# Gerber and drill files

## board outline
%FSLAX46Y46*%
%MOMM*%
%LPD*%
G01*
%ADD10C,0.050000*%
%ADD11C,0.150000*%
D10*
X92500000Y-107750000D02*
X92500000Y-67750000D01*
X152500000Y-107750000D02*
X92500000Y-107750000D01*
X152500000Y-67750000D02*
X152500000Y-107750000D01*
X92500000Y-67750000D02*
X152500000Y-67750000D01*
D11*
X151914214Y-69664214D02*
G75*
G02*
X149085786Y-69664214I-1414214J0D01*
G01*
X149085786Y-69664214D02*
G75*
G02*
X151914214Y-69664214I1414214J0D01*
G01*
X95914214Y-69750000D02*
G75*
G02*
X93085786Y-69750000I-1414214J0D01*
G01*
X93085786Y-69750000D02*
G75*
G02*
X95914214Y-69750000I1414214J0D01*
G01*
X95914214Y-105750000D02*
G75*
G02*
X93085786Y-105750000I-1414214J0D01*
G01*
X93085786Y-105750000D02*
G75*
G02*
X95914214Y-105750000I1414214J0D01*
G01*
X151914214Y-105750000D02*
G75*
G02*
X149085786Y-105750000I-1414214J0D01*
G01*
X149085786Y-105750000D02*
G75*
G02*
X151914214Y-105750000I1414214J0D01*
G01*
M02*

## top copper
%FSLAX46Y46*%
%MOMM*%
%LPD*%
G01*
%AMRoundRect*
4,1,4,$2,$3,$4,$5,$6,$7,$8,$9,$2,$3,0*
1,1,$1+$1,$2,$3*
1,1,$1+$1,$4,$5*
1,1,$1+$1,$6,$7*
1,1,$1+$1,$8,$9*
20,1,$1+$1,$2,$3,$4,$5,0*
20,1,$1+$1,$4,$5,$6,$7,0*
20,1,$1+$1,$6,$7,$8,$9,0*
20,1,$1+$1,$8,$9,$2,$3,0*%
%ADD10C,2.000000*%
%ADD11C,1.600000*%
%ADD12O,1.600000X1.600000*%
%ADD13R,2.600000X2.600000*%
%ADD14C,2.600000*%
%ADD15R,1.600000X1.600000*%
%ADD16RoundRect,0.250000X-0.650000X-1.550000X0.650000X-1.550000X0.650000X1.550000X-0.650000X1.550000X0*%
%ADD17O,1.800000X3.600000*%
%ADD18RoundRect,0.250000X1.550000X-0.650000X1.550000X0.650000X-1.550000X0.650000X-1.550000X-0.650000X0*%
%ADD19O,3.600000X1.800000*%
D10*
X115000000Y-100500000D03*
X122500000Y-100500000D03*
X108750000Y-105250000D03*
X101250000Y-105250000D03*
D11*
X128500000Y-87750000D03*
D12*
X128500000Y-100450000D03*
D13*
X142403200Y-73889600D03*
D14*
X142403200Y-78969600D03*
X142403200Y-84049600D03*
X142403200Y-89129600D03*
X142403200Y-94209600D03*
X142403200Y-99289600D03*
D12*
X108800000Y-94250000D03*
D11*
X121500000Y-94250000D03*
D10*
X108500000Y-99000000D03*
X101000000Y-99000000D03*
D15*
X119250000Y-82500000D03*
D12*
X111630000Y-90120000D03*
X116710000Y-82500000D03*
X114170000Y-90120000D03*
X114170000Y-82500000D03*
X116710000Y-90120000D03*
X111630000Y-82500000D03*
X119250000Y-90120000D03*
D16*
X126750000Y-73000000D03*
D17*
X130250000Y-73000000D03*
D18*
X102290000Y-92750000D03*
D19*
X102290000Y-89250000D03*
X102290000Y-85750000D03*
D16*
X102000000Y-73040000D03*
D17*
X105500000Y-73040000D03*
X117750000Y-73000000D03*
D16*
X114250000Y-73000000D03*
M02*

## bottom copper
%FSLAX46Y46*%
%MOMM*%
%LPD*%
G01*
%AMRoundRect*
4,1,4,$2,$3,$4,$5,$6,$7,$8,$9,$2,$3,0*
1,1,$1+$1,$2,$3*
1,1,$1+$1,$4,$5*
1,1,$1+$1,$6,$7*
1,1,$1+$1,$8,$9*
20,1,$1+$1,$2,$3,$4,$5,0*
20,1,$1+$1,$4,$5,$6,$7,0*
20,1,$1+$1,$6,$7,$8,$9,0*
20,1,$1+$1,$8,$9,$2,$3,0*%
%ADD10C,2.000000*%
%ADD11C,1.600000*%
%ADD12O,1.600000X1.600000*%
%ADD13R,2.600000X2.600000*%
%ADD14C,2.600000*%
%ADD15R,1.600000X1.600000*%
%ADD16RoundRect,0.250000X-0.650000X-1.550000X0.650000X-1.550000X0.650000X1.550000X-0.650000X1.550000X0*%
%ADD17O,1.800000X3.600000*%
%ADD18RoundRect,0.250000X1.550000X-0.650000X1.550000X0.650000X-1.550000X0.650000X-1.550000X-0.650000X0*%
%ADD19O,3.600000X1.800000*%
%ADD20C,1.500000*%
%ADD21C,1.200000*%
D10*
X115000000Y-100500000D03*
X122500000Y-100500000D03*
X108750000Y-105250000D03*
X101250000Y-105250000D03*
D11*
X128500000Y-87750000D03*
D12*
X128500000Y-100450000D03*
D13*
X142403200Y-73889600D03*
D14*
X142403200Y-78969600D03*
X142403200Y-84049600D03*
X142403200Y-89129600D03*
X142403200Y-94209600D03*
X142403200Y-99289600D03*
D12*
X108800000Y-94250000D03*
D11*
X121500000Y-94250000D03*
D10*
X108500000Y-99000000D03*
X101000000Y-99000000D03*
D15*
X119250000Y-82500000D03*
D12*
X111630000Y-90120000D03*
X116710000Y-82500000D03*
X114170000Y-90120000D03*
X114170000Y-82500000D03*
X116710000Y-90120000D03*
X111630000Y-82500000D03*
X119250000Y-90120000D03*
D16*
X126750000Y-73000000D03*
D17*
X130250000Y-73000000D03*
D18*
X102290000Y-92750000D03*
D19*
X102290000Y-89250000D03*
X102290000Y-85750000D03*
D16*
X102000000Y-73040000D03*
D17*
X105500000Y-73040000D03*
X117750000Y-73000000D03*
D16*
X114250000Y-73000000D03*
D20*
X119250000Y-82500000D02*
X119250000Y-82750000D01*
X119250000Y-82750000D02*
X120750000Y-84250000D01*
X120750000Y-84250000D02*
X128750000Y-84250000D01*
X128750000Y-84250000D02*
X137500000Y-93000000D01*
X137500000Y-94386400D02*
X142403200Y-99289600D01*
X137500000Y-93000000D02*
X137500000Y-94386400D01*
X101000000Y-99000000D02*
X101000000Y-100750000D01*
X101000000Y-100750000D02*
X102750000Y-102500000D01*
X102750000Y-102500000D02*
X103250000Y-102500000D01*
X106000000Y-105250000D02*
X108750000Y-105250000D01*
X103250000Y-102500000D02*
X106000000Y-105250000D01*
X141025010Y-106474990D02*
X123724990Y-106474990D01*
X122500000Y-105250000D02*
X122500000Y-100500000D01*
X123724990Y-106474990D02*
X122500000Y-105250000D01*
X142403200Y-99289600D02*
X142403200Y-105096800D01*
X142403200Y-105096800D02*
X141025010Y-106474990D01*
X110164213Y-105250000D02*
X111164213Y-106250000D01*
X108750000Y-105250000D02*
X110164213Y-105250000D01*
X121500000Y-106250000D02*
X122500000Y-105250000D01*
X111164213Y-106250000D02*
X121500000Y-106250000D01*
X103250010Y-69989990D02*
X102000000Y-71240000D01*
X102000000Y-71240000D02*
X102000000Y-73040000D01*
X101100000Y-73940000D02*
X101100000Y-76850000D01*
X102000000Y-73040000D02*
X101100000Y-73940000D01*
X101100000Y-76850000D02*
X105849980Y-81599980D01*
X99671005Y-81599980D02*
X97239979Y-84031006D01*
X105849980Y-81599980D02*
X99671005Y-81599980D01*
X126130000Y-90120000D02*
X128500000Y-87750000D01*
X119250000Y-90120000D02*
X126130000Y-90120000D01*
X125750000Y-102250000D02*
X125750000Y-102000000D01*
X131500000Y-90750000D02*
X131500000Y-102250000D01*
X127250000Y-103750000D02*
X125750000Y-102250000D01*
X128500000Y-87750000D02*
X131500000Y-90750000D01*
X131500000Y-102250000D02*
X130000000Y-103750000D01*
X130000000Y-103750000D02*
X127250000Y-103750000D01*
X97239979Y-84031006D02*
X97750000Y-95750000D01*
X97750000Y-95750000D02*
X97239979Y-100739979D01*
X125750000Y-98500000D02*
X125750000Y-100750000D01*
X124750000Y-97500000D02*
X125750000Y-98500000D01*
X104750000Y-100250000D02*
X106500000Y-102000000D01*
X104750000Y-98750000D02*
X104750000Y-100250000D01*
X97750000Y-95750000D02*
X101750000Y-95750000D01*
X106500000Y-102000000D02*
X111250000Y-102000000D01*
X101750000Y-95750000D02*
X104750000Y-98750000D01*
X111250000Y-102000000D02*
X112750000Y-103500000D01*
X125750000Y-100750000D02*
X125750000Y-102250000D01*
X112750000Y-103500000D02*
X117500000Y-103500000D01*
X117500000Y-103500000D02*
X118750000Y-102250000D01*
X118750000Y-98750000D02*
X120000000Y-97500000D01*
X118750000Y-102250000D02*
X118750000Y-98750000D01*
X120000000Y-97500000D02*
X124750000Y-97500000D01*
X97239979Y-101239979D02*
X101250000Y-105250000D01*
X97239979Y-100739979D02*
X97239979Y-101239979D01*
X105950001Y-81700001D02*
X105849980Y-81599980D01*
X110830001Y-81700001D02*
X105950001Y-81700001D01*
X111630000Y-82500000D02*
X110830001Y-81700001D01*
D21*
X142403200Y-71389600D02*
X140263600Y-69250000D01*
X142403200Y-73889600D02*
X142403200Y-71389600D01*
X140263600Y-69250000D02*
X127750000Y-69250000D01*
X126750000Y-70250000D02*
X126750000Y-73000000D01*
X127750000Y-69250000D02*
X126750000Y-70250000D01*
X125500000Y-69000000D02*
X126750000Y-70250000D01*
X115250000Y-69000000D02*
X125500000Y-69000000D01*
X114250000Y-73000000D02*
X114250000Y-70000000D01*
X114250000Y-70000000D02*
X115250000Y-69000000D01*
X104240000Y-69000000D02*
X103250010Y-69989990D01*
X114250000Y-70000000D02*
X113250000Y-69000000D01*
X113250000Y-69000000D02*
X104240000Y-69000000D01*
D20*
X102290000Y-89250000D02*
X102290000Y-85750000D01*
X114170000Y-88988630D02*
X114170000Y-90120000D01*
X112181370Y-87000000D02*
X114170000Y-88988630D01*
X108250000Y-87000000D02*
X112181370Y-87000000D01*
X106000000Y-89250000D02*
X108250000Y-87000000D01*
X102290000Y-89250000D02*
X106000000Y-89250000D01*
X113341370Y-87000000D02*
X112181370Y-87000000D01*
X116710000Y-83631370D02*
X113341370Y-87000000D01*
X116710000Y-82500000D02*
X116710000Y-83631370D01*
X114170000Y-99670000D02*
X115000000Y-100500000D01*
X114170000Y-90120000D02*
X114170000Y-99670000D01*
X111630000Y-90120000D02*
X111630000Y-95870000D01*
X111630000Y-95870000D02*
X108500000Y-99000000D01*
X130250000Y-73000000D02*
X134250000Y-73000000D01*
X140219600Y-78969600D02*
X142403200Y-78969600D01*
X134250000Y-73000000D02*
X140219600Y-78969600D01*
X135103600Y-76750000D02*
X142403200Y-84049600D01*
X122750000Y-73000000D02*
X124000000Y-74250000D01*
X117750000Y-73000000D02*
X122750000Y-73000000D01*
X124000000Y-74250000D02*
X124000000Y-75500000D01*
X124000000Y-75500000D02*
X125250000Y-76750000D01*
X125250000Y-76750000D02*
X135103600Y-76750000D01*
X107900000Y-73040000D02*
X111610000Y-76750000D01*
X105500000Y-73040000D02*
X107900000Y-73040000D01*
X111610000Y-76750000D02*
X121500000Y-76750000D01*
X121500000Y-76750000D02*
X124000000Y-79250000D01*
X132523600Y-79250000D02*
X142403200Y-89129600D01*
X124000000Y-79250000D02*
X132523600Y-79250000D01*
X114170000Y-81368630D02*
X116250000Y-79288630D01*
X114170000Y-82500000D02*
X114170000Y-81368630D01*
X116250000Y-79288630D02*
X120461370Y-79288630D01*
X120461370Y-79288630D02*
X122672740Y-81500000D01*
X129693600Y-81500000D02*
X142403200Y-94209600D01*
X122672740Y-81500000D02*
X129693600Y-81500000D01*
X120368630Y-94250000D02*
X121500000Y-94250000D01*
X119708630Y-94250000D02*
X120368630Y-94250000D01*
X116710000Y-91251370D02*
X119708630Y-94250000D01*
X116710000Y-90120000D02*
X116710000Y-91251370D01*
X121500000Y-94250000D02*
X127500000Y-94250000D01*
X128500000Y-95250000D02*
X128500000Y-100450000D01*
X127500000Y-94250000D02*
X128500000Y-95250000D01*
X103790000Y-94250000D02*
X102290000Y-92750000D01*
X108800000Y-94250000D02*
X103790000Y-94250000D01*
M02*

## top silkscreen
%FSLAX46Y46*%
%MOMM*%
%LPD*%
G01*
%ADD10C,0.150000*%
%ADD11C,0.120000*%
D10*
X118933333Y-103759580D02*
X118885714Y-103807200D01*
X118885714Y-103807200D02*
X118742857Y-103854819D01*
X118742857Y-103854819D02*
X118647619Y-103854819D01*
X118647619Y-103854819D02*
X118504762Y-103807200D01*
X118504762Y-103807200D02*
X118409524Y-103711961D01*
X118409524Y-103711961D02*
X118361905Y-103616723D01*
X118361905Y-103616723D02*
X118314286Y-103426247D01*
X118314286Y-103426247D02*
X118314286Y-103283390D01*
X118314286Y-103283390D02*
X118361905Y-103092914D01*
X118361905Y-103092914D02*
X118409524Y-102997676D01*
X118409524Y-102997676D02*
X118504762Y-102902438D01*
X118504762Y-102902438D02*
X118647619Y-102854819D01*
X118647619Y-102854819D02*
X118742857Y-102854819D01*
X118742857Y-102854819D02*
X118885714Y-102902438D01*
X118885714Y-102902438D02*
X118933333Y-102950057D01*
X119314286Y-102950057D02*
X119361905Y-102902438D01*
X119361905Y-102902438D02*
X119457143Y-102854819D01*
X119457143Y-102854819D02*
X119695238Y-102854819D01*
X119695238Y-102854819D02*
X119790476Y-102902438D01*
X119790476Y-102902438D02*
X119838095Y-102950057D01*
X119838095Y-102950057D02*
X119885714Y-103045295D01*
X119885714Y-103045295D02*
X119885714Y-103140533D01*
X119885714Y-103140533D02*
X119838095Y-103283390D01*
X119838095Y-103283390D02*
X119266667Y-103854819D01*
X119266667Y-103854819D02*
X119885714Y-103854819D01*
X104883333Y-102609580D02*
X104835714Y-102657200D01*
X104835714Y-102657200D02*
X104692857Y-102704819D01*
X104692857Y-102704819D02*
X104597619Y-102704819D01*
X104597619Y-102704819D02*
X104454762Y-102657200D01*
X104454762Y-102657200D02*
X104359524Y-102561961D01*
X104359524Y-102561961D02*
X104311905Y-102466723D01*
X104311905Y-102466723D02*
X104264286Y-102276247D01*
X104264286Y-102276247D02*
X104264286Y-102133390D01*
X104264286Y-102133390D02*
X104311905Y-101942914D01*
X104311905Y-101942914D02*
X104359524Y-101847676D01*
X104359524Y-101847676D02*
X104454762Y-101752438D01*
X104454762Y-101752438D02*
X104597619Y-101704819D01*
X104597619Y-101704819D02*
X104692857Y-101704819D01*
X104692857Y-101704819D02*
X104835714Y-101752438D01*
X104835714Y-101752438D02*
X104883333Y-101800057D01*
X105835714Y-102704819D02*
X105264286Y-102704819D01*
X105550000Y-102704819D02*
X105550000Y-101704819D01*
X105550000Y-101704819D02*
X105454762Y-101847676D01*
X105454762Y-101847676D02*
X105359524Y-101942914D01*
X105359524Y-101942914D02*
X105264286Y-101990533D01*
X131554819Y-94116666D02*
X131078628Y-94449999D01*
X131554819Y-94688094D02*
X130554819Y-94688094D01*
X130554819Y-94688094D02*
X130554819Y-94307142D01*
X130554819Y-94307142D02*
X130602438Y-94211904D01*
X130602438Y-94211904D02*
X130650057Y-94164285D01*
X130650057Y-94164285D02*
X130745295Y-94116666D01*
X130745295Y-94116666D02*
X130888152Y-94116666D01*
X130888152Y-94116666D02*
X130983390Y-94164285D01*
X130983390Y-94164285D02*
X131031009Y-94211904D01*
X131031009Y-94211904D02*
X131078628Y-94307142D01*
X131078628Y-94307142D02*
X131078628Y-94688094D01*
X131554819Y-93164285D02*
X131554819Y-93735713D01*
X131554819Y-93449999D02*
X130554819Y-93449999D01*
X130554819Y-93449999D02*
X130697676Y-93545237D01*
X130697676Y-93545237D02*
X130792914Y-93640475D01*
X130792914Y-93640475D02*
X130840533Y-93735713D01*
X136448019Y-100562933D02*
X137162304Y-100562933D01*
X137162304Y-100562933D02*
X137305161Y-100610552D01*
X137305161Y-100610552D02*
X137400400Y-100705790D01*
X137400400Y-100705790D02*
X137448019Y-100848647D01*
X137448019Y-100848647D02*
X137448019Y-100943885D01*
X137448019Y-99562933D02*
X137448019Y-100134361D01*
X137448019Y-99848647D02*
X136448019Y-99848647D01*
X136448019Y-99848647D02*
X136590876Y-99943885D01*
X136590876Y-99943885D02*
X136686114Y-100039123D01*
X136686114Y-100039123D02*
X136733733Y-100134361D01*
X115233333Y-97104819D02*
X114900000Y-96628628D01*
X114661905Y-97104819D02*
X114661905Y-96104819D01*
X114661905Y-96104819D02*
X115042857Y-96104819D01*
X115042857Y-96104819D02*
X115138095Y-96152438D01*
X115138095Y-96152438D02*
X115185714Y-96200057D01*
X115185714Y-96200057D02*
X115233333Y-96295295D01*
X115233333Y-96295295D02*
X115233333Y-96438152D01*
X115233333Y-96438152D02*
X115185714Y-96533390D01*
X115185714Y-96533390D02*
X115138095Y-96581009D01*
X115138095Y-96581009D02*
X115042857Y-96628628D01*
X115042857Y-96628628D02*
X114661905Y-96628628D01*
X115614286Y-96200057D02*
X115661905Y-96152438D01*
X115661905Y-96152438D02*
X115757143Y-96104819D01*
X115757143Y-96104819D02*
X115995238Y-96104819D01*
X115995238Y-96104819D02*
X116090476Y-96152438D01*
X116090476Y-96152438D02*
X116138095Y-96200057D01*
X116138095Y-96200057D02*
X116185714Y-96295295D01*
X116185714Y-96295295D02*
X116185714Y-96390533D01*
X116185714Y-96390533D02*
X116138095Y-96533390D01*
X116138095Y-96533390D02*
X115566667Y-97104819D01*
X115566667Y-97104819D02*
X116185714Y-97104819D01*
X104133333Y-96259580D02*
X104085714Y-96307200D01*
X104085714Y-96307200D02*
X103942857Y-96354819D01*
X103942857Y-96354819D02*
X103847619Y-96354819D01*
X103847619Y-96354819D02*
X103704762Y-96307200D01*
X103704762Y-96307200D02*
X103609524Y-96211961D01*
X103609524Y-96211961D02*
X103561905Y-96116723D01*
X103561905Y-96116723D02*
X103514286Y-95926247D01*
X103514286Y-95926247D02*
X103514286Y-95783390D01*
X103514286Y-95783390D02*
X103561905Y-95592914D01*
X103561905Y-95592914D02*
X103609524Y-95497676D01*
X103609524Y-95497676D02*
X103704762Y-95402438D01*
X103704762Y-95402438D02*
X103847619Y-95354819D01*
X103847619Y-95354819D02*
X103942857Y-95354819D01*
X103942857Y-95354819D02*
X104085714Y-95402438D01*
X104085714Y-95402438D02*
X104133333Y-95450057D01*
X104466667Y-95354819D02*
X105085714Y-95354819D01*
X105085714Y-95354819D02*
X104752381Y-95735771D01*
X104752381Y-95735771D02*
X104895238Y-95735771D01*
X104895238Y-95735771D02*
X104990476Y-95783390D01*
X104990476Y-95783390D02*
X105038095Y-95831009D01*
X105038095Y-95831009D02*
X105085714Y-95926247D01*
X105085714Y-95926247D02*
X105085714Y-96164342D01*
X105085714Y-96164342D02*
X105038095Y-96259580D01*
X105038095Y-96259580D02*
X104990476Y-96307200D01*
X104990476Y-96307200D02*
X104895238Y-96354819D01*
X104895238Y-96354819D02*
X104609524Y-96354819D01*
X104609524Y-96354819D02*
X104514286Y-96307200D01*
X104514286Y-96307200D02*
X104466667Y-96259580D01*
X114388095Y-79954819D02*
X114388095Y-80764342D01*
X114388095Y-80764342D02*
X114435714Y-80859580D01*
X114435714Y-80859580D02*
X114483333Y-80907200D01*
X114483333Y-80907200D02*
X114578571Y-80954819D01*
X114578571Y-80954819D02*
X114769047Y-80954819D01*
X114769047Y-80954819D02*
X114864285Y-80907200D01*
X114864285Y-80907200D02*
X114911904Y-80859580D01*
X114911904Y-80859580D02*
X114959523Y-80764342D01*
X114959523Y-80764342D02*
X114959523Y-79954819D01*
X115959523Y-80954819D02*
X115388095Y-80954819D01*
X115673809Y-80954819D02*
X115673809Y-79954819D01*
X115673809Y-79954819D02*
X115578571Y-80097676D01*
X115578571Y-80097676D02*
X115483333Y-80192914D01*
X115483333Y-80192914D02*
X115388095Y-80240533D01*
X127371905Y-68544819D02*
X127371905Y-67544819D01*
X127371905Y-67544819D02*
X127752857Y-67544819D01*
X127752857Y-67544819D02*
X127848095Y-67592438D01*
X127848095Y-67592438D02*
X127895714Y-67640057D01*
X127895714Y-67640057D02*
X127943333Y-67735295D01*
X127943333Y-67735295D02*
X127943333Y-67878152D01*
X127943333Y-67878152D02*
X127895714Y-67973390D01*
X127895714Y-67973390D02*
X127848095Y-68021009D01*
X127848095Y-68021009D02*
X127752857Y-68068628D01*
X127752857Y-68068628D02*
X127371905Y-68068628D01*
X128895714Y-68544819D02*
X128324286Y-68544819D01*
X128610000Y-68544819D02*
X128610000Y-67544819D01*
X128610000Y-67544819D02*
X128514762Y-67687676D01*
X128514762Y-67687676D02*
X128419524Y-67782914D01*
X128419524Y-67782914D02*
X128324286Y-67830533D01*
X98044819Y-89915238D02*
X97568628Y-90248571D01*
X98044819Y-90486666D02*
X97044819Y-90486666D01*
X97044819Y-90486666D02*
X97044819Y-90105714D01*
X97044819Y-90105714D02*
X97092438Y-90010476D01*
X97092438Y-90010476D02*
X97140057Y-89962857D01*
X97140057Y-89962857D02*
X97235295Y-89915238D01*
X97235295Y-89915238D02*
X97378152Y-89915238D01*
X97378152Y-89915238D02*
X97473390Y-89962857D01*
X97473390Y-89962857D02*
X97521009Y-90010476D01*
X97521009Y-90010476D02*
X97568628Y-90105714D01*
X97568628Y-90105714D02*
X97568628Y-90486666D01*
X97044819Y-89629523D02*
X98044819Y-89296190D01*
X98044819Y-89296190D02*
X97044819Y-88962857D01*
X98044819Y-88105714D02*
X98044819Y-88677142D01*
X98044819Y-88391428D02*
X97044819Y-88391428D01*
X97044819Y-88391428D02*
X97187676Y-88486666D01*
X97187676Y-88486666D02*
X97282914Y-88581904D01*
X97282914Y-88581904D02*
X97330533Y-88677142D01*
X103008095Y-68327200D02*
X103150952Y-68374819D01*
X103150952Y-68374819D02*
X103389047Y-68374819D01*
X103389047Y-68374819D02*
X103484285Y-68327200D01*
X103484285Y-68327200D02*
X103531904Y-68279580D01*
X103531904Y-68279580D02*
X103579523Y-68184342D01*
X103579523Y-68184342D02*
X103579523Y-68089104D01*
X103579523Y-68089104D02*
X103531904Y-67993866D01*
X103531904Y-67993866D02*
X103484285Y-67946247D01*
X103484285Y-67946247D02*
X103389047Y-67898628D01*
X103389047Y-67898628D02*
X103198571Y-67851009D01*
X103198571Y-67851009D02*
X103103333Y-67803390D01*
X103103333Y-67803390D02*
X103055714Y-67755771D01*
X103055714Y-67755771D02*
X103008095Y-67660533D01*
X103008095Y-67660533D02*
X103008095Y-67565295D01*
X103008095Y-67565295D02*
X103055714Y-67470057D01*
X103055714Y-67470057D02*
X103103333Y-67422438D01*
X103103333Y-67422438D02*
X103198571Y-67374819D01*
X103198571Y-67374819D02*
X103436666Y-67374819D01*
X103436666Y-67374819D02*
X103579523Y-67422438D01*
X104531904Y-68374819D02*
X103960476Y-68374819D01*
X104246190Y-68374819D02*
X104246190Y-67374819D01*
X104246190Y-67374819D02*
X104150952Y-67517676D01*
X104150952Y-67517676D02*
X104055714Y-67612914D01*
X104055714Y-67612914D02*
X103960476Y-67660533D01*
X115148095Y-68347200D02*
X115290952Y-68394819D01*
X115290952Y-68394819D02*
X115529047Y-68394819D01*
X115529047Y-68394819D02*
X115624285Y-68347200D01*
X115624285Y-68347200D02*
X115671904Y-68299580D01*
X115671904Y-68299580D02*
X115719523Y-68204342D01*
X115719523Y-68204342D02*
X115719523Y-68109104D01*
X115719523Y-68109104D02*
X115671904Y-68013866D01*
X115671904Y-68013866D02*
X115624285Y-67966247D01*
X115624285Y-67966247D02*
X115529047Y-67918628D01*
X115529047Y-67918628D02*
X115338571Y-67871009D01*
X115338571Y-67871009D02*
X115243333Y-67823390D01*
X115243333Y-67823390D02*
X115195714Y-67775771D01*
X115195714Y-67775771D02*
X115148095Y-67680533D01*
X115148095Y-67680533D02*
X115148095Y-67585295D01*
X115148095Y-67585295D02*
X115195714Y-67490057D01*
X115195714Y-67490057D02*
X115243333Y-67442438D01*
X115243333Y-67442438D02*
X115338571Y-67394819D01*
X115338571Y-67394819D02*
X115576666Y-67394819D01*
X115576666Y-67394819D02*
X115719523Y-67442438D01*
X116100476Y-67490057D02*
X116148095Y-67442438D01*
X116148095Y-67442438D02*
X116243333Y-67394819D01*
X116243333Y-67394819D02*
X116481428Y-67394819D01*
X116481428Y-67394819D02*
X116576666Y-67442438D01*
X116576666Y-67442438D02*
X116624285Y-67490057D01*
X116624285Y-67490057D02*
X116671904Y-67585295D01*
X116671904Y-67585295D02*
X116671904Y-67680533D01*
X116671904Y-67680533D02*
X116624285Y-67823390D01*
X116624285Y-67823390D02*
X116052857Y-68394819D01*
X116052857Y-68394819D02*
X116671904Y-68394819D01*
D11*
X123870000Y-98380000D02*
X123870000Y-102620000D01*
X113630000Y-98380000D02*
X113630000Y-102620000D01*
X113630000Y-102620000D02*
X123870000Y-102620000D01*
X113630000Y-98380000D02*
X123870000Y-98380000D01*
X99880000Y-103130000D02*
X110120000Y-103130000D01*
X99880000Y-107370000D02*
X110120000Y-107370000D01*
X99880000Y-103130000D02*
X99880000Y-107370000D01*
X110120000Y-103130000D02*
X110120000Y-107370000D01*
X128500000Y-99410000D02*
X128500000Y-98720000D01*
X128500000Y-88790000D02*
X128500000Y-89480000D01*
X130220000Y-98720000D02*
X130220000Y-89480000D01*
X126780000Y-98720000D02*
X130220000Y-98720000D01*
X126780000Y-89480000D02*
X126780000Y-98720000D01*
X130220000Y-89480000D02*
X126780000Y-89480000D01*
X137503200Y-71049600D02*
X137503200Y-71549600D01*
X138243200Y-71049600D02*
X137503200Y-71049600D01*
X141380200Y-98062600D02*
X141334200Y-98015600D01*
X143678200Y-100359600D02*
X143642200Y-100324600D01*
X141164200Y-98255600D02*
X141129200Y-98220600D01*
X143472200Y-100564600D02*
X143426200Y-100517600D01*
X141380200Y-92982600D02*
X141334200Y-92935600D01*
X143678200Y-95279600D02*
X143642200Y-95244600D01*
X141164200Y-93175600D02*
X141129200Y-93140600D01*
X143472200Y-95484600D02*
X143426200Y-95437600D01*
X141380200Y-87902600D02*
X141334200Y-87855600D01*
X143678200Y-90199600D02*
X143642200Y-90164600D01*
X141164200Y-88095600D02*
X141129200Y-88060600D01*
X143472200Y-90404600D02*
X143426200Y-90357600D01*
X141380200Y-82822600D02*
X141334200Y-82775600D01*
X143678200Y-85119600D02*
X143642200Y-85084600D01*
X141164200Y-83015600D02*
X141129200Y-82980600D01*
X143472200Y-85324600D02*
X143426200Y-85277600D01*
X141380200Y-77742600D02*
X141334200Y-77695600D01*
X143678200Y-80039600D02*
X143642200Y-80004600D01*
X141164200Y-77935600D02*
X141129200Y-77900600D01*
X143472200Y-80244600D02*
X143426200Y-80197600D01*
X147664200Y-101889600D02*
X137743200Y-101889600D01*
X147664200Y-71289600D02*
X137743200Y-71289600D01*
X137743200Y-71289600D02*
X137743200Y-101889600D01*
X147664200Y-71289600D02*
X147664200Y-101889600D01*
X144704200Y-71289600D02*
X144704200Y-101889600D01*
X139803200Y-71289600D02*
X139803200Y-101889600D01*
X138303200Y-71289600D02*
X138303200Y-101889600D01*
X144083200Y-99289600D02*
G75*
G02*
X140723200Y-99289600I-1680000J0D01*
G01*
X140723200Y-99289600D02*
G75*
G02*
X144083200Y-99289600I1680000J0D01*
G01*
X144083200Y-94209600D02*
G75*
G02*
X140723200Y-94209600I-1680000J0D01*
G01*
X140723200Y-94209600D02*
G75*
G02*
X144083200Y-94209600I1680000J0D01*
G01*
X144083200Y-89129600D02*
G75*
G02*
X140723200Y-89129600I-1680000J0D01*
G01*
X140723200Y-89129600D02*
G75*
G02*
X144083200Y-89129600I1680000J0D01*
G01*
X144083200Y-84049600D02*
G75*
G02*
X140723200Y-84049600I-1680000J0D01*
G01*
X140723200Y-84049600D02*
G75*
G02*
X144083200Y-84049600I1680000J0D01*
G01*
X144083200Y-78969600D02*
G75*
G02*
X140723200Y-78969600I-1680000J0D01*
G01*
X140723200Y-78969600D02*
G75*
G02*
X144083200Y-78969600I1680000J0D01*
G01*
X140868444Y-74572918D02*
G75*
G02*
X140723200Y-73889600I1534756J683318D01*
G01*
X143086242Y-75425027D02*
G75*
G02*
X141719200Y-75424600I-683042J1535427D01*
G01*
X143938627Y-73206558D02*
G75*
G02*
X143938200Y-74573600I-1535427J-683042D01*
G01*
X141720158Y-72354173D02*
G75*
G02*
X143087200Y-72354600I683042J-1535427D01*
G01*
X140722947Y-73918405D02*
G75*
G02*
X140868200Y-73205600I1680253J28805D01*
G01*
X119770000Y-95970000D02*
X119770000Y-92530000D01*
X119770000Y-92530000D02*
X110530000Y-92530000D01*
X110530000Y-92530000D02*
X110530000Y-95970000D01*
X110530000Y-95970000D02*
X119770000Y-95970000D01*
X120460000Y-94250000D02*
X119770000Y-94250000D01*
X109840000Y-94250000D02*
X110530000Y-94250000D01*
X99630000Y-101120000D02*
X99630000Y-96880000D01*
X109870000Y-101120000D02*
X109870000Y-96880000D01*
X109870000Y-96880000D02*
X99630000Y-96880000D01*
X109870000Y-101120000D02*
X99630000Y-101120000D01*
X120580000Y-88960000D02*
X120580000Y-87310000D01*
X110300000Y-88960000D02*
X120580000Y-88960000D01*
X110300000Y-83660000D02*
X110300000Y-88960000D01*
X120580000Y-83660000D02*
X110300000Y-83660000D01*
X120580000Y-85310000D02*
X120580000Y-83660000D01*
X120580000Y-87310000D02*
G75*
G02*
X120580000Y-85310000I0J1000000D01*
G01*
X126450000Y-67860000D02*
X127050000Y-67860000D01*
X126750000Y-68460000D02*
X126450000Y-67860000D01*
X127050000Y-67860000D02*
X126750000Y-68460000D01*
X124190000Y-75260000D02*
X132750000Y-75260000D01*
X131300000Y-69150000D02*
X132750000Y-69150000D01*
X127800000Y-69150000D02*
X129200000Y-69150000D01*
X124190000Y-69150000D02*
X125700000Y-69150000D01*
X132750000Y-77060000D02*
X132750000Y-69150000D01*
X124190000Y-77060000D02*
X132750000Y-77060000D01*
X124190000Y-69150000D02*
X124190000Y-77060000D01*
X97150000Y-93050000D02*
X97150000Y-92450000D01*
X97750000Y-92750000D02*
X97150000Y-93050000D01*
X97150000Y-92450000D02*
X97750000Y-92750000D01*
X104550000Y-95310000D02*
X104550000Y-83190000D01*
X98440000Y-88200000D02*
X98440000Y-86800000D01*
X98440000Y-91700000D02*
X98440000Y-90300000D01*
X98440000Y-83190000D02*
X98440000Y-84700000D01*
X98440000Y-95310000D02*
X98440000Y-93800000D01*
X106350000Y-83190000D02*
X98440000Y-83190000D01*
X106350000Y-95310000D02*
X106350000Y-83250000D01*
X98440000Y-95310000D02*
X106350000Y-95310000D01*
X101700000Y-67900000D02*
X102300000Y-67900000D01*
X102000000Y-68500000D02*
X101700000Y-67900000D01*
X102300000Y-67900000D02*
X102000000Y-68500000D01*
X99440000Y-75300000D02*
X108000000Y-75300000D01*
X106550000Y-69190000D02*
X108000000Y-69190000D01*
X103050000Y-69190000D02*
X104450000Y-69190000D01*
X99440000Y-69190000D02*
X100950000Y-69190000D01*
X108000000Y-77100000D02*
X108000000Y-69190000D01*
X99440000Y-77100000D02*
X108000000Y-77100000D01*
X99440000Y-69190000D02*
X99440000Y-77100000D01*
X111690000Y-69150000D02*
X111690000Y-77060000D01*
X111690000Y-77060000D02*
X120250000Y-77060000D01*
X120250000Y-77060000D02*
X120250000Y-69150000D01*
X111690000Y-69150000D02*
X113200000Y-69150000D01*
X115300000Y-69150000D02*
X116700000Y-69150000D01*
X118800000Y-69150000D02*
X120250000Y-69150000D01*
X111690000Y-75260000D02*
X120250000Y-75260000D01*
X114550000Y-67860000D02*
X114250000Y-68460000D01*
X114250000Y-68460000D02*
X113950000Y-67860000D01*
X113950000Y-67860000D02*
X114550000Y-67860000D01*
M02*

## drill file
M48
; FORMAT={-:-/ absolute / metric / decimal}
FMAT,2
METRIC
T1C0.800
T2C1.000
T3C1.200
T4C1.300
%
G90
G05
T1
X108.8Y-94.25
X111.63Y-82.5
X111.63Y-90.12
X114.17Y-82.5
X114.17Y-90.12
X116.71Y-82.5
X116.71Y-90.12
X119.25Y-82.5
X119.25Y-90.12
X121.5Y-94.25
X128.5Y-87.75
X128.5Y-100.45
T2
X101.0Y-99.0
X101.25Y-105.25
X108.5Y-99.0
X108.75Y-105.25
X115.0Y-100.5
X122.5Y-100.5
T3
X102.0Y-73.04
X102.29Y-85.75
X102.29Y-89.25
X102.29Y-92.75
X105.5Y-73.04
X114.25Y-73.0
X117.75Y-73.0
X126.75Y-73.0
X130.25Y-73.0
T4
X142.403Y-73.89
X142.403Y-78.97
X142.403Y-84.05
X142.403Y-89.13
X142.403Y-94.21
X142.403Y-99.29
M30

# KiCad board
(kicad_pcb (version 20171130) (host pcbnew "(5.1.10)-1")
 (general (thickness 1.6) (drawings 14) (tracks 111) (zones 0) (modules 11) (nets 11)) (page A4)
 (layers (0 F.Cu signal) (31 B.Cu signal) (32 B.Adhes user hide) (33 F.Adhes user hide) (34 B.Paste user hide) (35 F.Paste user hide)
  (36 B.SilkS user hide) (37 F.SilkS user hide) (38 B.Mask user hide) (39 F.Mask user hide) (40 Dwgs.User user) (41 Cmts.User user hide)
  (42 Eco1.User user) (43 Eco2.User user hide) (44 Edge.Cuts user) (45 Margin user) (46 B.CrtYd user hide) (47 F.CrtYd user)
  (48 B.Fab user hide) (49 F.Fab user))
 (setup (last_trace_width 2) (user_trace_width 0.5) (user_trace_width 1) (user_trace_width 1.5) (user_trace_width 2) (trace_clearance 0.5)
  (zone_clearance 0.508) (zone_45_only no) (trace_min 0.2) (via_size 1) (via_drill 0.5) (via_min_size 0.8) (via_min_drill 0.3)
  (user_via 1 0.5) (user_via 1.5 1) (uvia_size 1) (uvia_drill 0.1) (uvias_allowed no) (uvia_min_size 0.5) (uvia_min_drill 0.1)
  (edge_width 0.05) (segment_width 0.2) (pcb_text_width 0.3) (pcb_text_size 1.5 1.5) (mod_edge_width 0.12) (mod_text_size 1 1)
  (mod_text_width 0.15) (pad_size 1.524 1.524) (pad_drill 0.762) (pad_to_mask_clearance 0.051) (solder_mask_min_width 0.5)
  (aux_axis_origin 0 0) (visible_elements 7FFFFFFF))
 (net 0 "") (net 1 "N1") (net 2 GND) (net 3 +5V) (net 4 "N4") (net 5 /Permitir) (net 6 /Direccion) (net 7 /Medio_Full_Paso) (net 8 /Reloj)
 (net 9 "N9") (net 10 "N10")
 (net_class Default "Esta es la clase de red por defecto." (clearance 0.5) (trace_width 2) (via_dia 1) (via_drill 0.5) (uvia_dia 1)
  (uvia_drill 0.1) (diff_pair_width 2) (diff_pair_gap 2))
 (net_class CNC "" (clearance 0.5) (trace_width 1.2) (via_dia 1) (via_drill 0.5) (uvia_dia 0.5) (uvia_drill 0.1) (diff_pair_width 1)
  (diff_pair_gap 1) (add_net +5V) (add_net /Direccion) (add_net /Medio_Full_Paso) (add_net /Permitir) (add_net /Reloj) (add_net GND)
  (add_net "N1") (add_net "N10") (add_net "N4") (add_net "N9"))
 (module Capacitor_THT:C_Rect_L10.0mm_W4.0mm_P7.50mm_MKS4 (layer F.Cu) (at 115 100.5)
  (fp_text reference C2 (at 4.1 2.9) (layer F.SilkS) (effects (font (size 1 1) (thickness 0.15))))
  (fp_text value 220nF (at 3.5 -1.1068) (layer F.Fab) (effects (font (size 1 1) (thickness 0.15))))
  (fp_line (start 8.87 -2.12) (end 8.87 2.12) (layer F.SilkS) (width 0.12))
  (fp_line (start -1.37 -2.12) (end -1.37 2.12) (layer F.SilkS) (width 0.12))
  (fp_line (start -1.37 2.12) (end 8.87 2.12) (layer F.SilkS) (width 0.12))
  (fp_line (start -1.37 -2.12) (end 8.87 -2.12) (layer F.SilkS) (width 0.12))
  (pad 1 thru_hole circle (at 0 0) (size 2 2) (drill 1) (layers *.Cu *.Mask) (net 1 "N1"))
  (pad 2 thru_hole circle (at 7.5 0) (size 2 2) (drill 1) (layers *.Cu *.Mask) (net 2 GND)))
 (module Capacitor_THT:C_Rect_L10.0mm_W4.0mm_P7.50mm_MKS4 (layer F.Cu) (at 101.25 105.25)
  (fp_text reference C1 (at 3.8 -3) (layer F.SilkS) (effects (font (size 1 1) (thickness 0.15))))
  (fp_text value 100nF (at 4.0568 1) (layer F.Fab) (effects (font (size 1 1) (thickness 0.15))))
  (fp_line (start -1.37 -2.12) (end 8.87 -2.12) (layer F.SilkS) (width 0.12))
  (fp_line (start -1.37 2.12) (end 8.87 2.12) (layer F.SilkS) (width 0.12))
  (fp_line (start -1.37 -2.12) (end -1.37 2.12) (layer F.SilkS) (width 0.12))
  (fp_line (start 8.87 -2.12) (end 8.87 2.12) (layer F.SilkS) (width 0.12))
  (pad 2 thru_hole circle (at 7.5 0) (size 2 2) (drill 1) (layers *.Cu *.Mask) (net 2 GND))
  (pad 1 thru_hole circle (at 0 0) (size 2 2) (drill 1) (layers *.Cu *.Mask) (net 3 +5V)))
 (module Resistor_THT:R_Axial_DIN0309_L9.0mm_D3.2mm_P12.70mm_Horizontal (layer F.Cu) (at 128.5 87.75 270)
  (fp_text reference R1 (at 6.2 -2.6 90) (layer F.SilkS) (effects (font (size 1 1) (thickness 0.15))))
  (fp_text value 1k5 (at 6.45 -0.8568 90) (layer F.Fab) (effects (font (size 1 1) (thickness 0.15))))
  (fp_line (start 11.66 0) (end 10.97 0) (layer F.SilkS) (width 0.12))
  (fp_line (start 1.04 0) (end 1.73 0) (layer F.SilkS) (width 0.12))
  (fp_line (start 10.97 -1.72) (end 1.73 -1.72) (layer F.SilkS) (width 0.12))
  (fp_line (start 10.97 1.72) (end 10.97 -1.72) (layer F.SilkS) (width 0.12))
  (fp_line (start 1.73 1.72) (end 10.97 1.72) (layer F.SilkS) (width 0.12))
  (fp_line (start 1.73 -1.72) (end 1.73 1.72) (layer F.SilkS) (width 0.12))
  (pad 1 thru_hole circle (at 0 0 270) (size 1.6 1.6) (drill 0.8) (layers *.Cu *.Mask) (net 3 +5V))
  (pad 2 thru_hole oval (at 12.7 0 270) (size 1.6 1.6) (drill 0.8) (layers *.Cu *.Mask) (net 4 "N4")))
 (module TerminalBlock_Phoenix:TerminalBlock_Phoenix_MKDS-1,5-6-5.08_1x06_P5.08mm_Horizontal (layer F.Cu) (at 142.4032 73.8896 270)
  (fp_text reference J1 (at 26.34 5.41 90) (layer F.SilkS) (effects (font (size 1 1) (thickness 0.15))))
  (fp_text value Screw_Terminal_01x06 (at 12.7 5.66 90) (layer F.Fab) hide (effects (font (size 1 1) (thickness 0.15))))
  (fp_line (start -2.84 4.9) (end -2.34 4.9) (layer F.SilkS) (width 0.12))
  (fp_line (start -2.84 4.16) (end -2.84 4.9) (layer F.SilkS) (width 0.12))
  (fp_line (start 24.173 1.023) (end 24.126 1.069) (layer F.SilkS) (width 0.12))
  (fp_line (start 26.47 -1.275) (end 26.435 -1.239) (layer F.SilkS) (width 0.12))
  (fp_line (start 24.366 1.239) (end 24.331 1.274) (layer F.SilkS) (width 0.12))
  (fp_line (start 26.675 -1.069) (end 26.628 -1.023) (layer F.SilkS) (width 0.12))
  (fp_line (start 19.093 1.023) (end 19.046 1.069) (layer F.SilkS) (width 0.12))
  (fp_line (start 21.39 -1.275) (end 21.355 -1.239) (layer F.SilkS) (width 0.12))
  (fp_line (start 19.286 1.239) (end 19.251 1.274) (layer F.SilkS) (width 0.12))
  (fp_line (start 21.595 -1.069) (end 21.548 -1.023) (layer F.SilkS) (width 0.12))
  (fp_line (start 14.013 1.023) (end 13.966 1.069) (layer F.SilkS) (width 0.12))
  (fp_line (start 16.31 -1.275) (end 16.275 -1.239) (layer F.SilkS) (width 0.12))
  (fp_line (start 14.206 1.239) (end 14.171 1.274) (layer F.SilkS) (width 0.12))
  (fp_line (start 16.515 -1.069) (end 16.468 -1.023) (layer F.SilkS) (width 0.12))
  (fp_line (start 8.933 1.023) (end 8.886 1.069) (layer F.SilkS) (width 0.12))
  (fp_line (start 11.23 -1.275) (end 11.195 -1.239) (layer F.SilkS) (width 0.12))
  (fp_line (start 9.126 1.239) (end 9.091 1.274) (layer F.SilkS) (width 0.12))
  (fp_line (start 11.435 -1.069) (end 11.388 -1.023) (layer F.SilkS) (width 0.12))
  (fp_line (start 3.853 1.023) (end 3.806 1.069) (layer F.SilkS) (width 0.12))
  (fp_line (start 6.15 -1.275) (end 6.115 -1.239) (layer F.SilkS) (width 0.12))
  (fp_line (start 4.046 1.239) (end 4.011 1.274) (layer F.SilkS) (width 0.12))
  (fp_line (start 6.355 -1.069) (end 6.308 -1.023) (layer F.SilkS) (width 0.12))
  (fp_line (start 28 -5.261) (end 28 4.66) (layer F.SilkS) (width 0.12))
  (fp_line (start -2.6 -5.261) (end -2.6 4.66) (layer F.SilkS) (width 0.12))
  (fp_line (start -2.6 4.66) (end 28 4.66) (layer F.SilkS) (width 0.12))
  (fp_line (start -2.6 -5.261) (end 28 -5.261) (layer F.SilkS) (width 0.12))
  (fp_line (start -2.6 -2.301) (end 28 -2.301) (layer F.SilkS) (width 0.12))
  (fp_line (start -2.6 2.6) (end 28 2.6) (layer F.SilkS) (width 0.12))
  (fp_line (start -2.6 4.1) (end 28 4.1) (layer F.SilkS) (width 0.12))
  (fp_circle (center 25.4 0) (end 27.08 0) (layer F.SilkS) (width 0.12))
  (fp_circle (center 20.32 0) (end 22 0) (layer F.SilkS) (width 0.12))
  (fp_circle (center 15.24 0) (end 16.92 0) (layer F.SilkS) (width 0.12))
  (fp_circle (center 10.16 0) (end 11.84 0) (layer F.SilkS) (width 0.12))
  (fp_circle (center 5.08 0) (end 6.76 0) (layer F.SilkS) (width 0.12))
  (fp_arc (start 0 0) (end 0 1.68) (angle -24) (layer F.SilkS) (width 0.12))
  (fp_arc (start 0 0) (end 1.535 0.684) (angle -48) (layer F.SilkS) (width 0.12))
  (fp_arc (start 0 0) (end 0.684 -1.535) (angle -48) (layer F.SilkS) (width 0.12))
  (fp_arc (start 0 0) (end -1.535 -0.684) (angle -48) (layer F.SilkS) (width 0.12))
  (fp_arc (start 0 0) (end -0.684 1.535) (angle -25) (layer F.SilkS) (width 0.12))
  (pad 1 thru_hole rect (at 0 0 270) (size 2.6 2.6) (drill 1.3) (layers *.Cu *.Mask) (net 3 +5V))
  (pad 2 thru_hole circle (at 5.08 0 270) (size 2.6 2.6) (drill 1.3) (layers *.Cu *.Mask) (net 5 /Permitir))
  (pad 3 thru_hole circle (at 10.16 0 270) (size 2.6 2.6) (drill 1.3) (layers *.Cu *.Mask) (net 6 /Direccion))
  (pad 4 thru_hole circle (at 15.24 0 270) (size 2.6 2.6) (drill 1.3) (layers *.Cu *.Mask) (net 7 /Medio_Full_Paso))
  (pad 5 thru_hole circle (at 20.32 0 270) (size 2.6 2.6) (drill 1.3) (layers *.Cu *.Mask) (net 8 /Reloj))
  (pad 6 thru_hole circle (at 25.4 0 270) (size 2.6 2.6) (drill 1.3) (layers *.Cu *.Mask) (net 2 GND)))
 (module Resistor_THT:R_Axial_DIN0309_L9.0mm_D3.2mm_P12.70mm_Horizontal (layer F.Cu) (at 121.5 94.25 180)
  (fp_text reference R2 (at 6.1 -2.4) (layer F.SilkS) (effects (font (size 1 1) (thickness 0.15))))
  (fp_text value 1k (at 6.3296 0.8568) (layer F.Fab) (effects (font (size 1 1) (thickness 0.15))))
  (fp_line (start 1.73 -1.72) (end 1.73 1.72) (layer F.SilkS) (width 0.12))
  (fp_line (start 1.73 1.72) (end 10.97 1.72) (layer F.SilkS) (width 0.12))
  (fp_line (start 10.97 1.72) (end 10.97 -1.72) (layer F.SilkS) (width 0.12))
  (fp_line (start 10.97 -1.72) (end 1.73 -1.72) (layer F.SilkS) (width 0.12))
  (fp_line (start 1.04 0) (end 1.73 0) (layer F.SilkS) (width 0.12))
  (fp_line (start 11.66 0) (end 10.97 0) (layer F.SilkS) (width 0.12))
  (pad 2 thru_hole oval (at 12.7 0 180) (size 1.6 1.6) (drill 0.8) (layers *.Cu *.Mask) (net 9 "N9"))
  (pad 1 thru_hole circle (at 0 0 180) (size 1.6 1.6) (drill 0.8) (layers *.Cu *.Mask) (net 4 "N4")))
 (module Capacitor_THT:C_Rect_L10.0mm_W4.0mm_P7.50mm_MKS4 (layer F.Cu) (at 108.5 99 180)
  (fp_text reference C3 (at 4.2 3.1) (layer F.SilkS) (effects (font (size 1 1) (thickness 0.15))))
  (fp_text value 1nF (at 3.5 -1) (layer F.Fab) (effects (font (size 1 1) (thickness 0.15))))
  (fp_line (start 8.87 -2.12) (end 8.87 2.12) (layer F.SilkS) (width 0.12))
  (fp_line (start -1.37 -2.12) (end -1.37 2.12) (layer F.SilkS) (width 0.12))
  (fp_line (start -1.37 2.12) (end 8.87 2.12) (layer F.SilkS) (width 0.12))
  (fp_line (start -1.37 -2.12) (end 8.87 -2.12) (layer F.SilkS) (width 0.12))
  (pad 1 thru_hole circle (at 0 0 180) (size 2 2) (drill 1) (layers *.Cu *.Mask) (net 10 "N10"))
  (pad 2 thru_hole circle (at 7.5 0 180) (size 2 2) (drill 1) (layers *.Cu *.Mask) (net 2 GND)))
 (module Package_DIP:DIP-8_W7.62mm (layer F.Cu) (at 119.25 82.5 270)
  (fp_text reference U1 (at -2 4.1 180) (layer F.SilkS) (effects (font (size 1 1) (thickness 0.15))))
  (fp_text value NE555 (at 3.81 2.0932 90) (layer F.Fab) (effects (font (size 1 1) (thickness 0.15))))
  (fp_line (start 6.46 -1.33) (end 4.81 -1.33) (layer F.SilkS) (width 0.12))
  (fp_line (start 6.46 8.95) (end 6.46 -1.33) (layer F.SilkS) (width 0.12))
  (fp_line (start 1.16 8.95) (end 6.46 8.95) (layer F.SilkS) (width 0.12))
  (fp_line (start 1.16 -1.33) (end 1.16 8.95) (layer F.SilkS) (width 0.12))
  (fp_line (start 2.81 -1.33) (end 1.16 -1.33) (layer F.SilkS) (width 0.12))
  (fp_arc (start 3.81 -1.33) (end 2.81 -1.33) (angle -180) (layer F.SilkS) (width 0.12))
  (pad 1 thru_hole rect (at 0 0 270) (size 1.6 1.6) (drill 0.8) (layers *.Cu *.Mask) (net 2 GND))
  (pad 5 thru_hole oval (at 7.62 7.62 270) (size 1.6 1.6) (drill 0.8) (layers *.Cu *.Mask) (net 10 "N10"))
  (pad 2 thru_hole oval (at 0 2.54 270) (size 1.6 1.6) (drill 0.8) (layers *.Cu *.Mask) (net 1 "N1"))
  (pad 6 thru_hole oval (at 7.62 5.08 270) (size 1.6 1.6) (drill 0.8) (layers *.Cu *.Mask) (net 1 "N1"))
  (pad 3 thru_hole oval (at 0 5.08 270) (size 1.6 1.6) (drill 0.8) (layers *.Cu *.Mask) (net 8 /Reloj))
  (pad 7 thru_hole oval (at 7.62 2.54 270) (size 1.6 1.6) (drill 0.8) (layers *.Cu *.Mask) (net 4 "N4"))
  (pad 4 thru_hole oval (at 0 7.62 270) (size 1.6 1.6) (drill 0.8) (layers *.Cu *.Mask) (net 3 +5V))
  (pad 8 thru_hole oval (at 7.62 0 270) (size 1.6 1.6) (drill 0.8) (layers *.Cu *.Mask) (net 3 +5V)))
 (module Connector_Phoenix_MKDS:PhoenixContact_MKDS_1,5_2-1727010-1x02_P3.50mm (layer F.Cu) (at 126.75 70.46)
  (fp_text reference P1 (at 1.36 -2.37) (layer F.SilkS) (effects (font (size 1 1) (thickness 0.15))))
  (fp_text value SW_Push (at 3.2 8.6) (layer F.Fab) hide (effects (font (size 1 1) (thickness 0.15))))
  (fp_line (start -0.3 -2.6) (end 0.3 -2.6) (layer F.SilkS) (width 0.12))
  (fp_line (start 0 -2) (end -0.3 -2.6) (layer F.SilkS) (width 0.12))
  (fp_line (start 0.3 -2.6) (end 0 -2) (layer F.SilkS) (width 0.12))
  (fp_line (start -2.56 4.8) (end 6 4.8) (layer F.SilkS) (width 0.12))
  (fp_line (start 4.55 -1.31) (end 6 -1.31) (layer F.SilkS) (width 0.12))
  (fp_line (start 1.05 -1.31) (end 2.45 -1.31) (layer F.SilkS) (width 0.12))
  (fp_line (start -2.56 -1.31) (end -1.05 -1.31) (layer F.SilkS) (width 0.12))
  (fp_line (start 6 6.6) (end 6 -1.31) (layer F.SilkS) (width 0.12))
  (fp_line (start -2.56 6.6) (end 6 6.6) (layer F.SilkS) (width 0.12))
  (fp_line (start -2.56 -1.31) (end -2.56 6.6) (layer F.SilkS) (width 0.12))
  (pad 1 thru_hole roundrect (at 0 2.54) (size 1.8 3.6) (drill 1.2) (layers *.Cu *.Mask) (roundrect_rratio 0.138889) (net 3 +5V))
  (pad 2 thru_hole oval (at 3.5 2.54) (size 1.8 3.6) (drill 1.2) (layers *.Cu *.Mask) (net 5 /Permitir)))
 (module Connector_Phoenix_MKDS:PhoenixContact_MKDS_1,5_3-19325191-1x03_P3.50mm (layer F.Cu) (at 99.75 92.75 90)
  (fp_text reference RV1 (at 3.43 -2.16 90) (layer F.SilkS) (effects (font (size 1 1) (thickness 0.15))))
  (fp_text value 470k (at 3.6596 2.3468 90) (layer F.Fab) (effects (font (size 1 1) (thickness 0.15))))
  (fp_line (start -0.3 -2.6) (end 0.3 -2.6) (layer F.SilkS) (width 0.12))
  (fp_line (start 0 -2) (end -0.3 -2.6) (layer F.SilkS) (width 0.12))
  (fp_line (start 0.3 -2.6) (end 0 -2) (layer F.SilkS) (width 0.12))
  (fp_line (start -2.56 4.8) (end 9.56 4.8) (layer F.SilkS) (width 0.12))
  (fp_line (start 4.55 -1.31) (end 5.95 -1.31) (layer F.SilkS) (width 0.12))
  (fp_line (start 1.05 -1.31) (end 2.45 -1.31) (layer F.SilkS) (width 0.12))
  (fp_line (start 9.56 -1.31) (end 8.05 -1.31) (layer F.SilkS) (width 0.12))
  (fp_line (start -2.56 -1.31) (end -1.05 -1.31) (layer F.SilkS) (width 0.12))
  (fp_line (start 9.56 6.6) (end 9.56 -1.31) (layer F.SilkS) (width 0.12))
  (fp_line (start -2.56 6.6) (end 9.5 6.6) (layer F.SilkS) (width 0.12))
  (fp_line (start -2.56 -1.31) (end -2.56 6.6) (layer F.SilkS) (width 0.12))
  (pad 1 thru_hole roundrect (at 0 2.54 90) (size 1.8 3.6) (drill 1.2) (layers *.Cu *.Mask) (roundrect_rratio 0.138889) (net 9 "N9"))
  (pad 2 thru_hole oval (at 3.5 2.54 90) (size 1.8 3.6) (drill 1.2) (layers *.Cu *.Mask) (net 1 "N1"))
  (pad 3 thru_hole oval (at 7 2.54 90) (size 1.8 3.6) (drill 1.2) (layers *.Cu *.Mask) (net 1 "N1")))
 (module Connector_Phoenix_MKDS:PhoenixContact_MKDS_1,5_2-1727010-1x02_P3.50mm (layer F.Cu) (at 102 70.5)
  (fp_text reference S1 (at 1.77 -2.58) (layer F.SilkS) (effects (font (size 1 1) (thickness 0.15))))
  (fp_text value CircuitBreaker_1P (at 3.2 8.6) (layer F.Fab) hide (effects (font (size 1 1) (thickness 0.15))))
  (fp_line (start -0.3 -2.6) (end 0.3 -2.6) (layer F.SilkS) (width 0.12))
  (fp_line (start 0 -2) (end -0.3 -2.6) (layer F.SilkS) (width 0.12))
  (fp_line (start 0.3 -2.6) (end 0 -2) (layer F.SilkS) (width 0.12))
  (fp_line (start -2.56 4.8) (end 6 4.8) (layer F.SilkS) (width 0.12))
  (fp_line (start 4.55 -1.31) (end 6 -1.31) (layer F.SilkS) (width 0.12))
  (fp_line (start 1.05 -1.31) (end 2.45 -1.31) (layer F.SilkS) (width 0.12))
  (fp_line (start -2.56 -1.31) (end -1.05 -1.31) (layer F.SilkS) (width 0.12))
  (fp_line (start 6 6.6) (end 6 -1.31) (layer F.SilkS) (width 0.12))
  (fp_line (start -2.56 6.6) (end 6 6.6) (layer F.SilkS) (width 0.12))
  (fp_line (start -2.56 -1.31) (end -2.56 6.6) (layer F.SilkS) (width 0.12))
  (pad 1 thru_hole roundrect (at 0 2.54) (size 1.8 3.6) (drill 1.2) (layers *.Cu *.Mask) (roundrect_rratio 0.138889) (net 3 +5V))
  (pad 2 thru_hole oval (at 3.5 2.54) (size 1.8 3.6) (drill 1.2) (layers *.Cu *.Mask) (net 7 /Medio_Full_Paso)))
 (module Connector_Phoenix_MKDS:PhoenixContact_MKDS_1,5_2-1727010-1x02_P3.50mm (layer F.Cu) (at 114.25 70.46)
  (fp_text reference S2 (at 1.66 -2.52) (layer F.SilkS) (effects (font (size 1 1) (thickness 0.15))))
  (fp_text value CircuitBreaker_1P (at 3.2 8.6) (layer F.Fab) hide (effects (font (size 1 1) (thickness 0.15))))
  (fp_line (start -2.56 -1.31) (end -2.56 6.6) (layer F.SilkS) (width 0.12))
  (fp_line (start -2.56 6.6) (end 6 6.6) (layer F.SilkS) (width 0.12))
  (fp_line (start 6 6.6) (end 6 -1.31) (layer F.SilkS) (width 0.12))
  (fp_line (start -2.56 -1.31) (end -1.05 -1.31) (layer F.SilkS) (width 0.12))
  (fp_line (start 1.05 -1.31) (end 2.45 -1.31) (layer F.SilkS) (width 0.12))
  (fp_line (start 4.55 -1.31) (end 6 -1.31) (layer F.SilkS) (width 0.12))
  (fp_line (start -2.56 4.8) (end 6 4.8) (layer F.SilkS) (width 0.12))
  (fp_line (start 0.3 -2.6) (end 0 -2) (layer F.SilkS) (width 0.12))
  (fp_line (start 0 -2) (end -0.3 -2.6) (layer F.SilkS) (width 0.12))
  (fp_line (start -0.3 -2.6) (end 0.3 -2.6) (layer F.SilkS) (width 0.12))
  (pad 2 thru_hole oval (at 3.5 2.54) (size 1.8 3.6) (drill 1.2) (layers *.Cu *.Mask) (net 6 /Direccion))
  (pad 1 thru_hole roundrect (at 0 2.54) (size 1.8 3.6) (drill 1.2) (layers *.Cu *.Mask) (roundrect_rratio 0.138889) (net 3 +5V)))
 (gr_line (start 92.5 107.75) (end 92.5 67.75) (layer Edge.Cuts) (width 0.05))
 (gr_line (start 152.5 107.75) (end 92.5 107.75) (layer Edge.Cuts) (width 0.05))
 (gr_line (start 152.5 67.75) (end 152.5 107.75) (layer Edge.Cuts) (width 0.05))
 (gr_line (start 92.5 67.75) (end 152.5 67.75) (layer Edge.Cuts) (width 0.05))
 (gr_circle (center 150.5 69.664214) (end 151.914214 69.664214) (layer Edge.Cuts) (width 0.15))
 (gr_circle (center 94.5 69.75) (end 95.914214 69.75) (layer Edge.Cuts) (width 0.15))
 (gr_circle (center 94.5 105.75) (end 95.914214 105.75) (layer Edge.Cuts) (width 0.15))
 (gr_circle (center 150.5 105.75) (end 151.914214 105.75) (layer Edge.Cuts) (width 0.15))
 (segment (start 119.25 82.5) (end 119.25 82.75) (width 1.5) (layer B.Cu) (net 2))
 (segment (start 119.25 82.75) (end 120.75 84.25) (width 1.5) (layer B.Cu) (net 2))
 (segment (start 120.75 84.25) (end 128.75 84.25) (width 1.5) (layer B.Cu) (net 2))
 (segment (start 128.75 84.25) (end 137.5 93) (width 1.5) (layer B.Cu) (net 2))
 (segment (start 137.5 94.3864) (end 142.4032 99.2896) (width 1.5) (layer B.Cu) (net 2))
 (segment (start 137.5 93) (end 137.5 94.3864) (width 1.5) (layer B.Cu) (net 2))
 (segment (start 101 99) (end 101 100.75) (width 1.5) (layer B.Cu) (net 2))
 (segment (start 101 100.75) (end 102.75 102.5) (width 1.5) (layer B.Cu) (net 2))
 (segment (start 102.75 102.5) (end 103.25 102.5) (width 1.5) (layer B.Cu) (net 2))
 (segment (start 106 105.25) (end 108.75 105.25) (width 1.5) (layer B.Cu) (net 2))
 (segment (start 103.25 102.5) (end 106 105.25) (width 1.5) (layer B.Cu) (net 2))
 (segment (start 141.02501 106.47499) (end 123.72499 106.47499) (width 1.5) (layer B.Cu) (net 2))
 (segment (start 122.5 105.25) (end 122.5 100.5) (width 1.5) (layer B.Cu) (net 2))
 (segment (start 123.72499 106.47499) (end 122.5 105.25) (width 1.5) (layer B.Cu) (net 2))
 (segment (start 142.4032 99.2896) (end 142.4032 105.0968) (width 1.5) (layer B.Cu) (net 2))
 (segment (start 142.4032 105.0968) (end 141.02501 106.47499) (width 1.5) (layer B.Cu) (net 2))
 (segment (start 110.164213 105.25) (end 111.164213 106.25) (width 1.5) (layer B.Cu) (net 2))
 (segment (start 108.75 105.25) (end 110.164213 105.25) (width 1.5) (layer B.Cu) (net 2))
 (segment (start 121.5 106.25) (end 122.5 105.25) (width 1.5) (layer B.Cu) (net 2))
 (segment (start 111.164213 106.25) (end 121.5 106.25) (width 1.5) (layer B.Cu) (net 2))
 (segment (start 103.25001 69.98999) (end 102 71.24) (width 1.5) (layer B.Cu) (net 3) (status 20))
 (segment (start 102 71.24) (end 102 73.04) (width 1.5) (layer B.Cu) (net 3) (status 30))
 (segment (start 101.1 73.94) (end 101.1 76.85) (width 1.5) (layer B.Cu) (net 3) (status 10))
 (segment (start 102 73.04) (end 101.1 73.94) (width 1.5) (layer B.Cu) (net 3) (status 30))
 (segment (start 101.1 76.85) (end 105.84998 81.59998) (width 1.5) (layer B.Cu) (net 3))
 (segment (start 99.671005 81.59998) (end 97.239979 84.031006) (width 1.5) (layer B.Cu) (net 3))
 (segment (start 105.84998 81.59998) (end 99.671005 81.59998) (width 1.5) (layer B.Cu) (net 3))
 (segment (start 126.13 90.12) (end 128.5 87.75) (width 1.5) (layer B.Cu) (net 3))
 (segment (start 119.25 90.12) (end 126.13 90.12) (width 1.5) (layer B.Cu) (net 3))
 (segment (start 125.75 102.25) (end 125.75 102) (width 1.5) (layer B.Cu) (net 3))
 (segment (start 131.5 90.75) (end 131.5 102.25) (width 1.5) (layer B.Cu) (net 3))
 (segment (start 127.25 103.75) (end 125.75 102.25) (width 1.5) (layer B.Cu) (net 3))
 (segment (start 128.5 87.75) (end 131.5 90.75) (width 1.5) (layer B.Cu) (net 3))
 (segment (start 131.5 102.25) (end 130 103.75) (width 1.5) (layer B.Cu) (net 3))
 (segment (start 130 103.75) (end 127.25 103.75) (width 1.5) (layer B.Cu) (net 3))
 (segment (start 97.239979 84.031006) (end 97.75 95.75) (width 1.5) (layer B.Cu) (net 3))
 (segment (start 97.75 95.75) (end 97.239979 100.739979) (width 1.5) (layer B.Cu) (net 3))
 (segment (start 125.75 98.5) (end 125.75 100.75) (width 1.5) (layer B.Cu) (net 3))
 (segment (start 124.75 97.5) (end 125.75 98.5) (width 1.5) (layer B.Cu) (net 3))
 (segment (start 104.75 100.25) (end 106.5 102) (width 1.5) (layer B.Cu) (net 3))
 (segment (start 104.75 98.75) (end 104.75 100.25) (width 1.5) (layer B.Cu) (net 3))
 (segment (start 97.75 95.75) (end 101.75 95.75) (width 1.5) (layer B.Cu) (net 3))
 (segment (start 106.5 102) (end 111.25 102) (width 1.5) (layer B.Cu) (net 3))
 (segment (start 101.75 95.75) (end 104.75 98.75) (width 1.5) (layer B.Cu) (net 3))
 (segment (start 111.25 102) (end 112.75 103.5) (width 1.5) (layer B.Cu) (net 3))
 (segment (start 125.75 100.75) (end 125.75 102.25) (width 1.5) (layer B.Cu) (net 3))
 (segment (start 112.75 103.5) (end 117.5 103.5) (width 1.5) (layer B.Cu) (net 3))
 (segment (start 117.5 103.5) (end 118.75 102.25) (width 1.5) (layer B.Cu) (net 3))
 (segment (start 118.75 98.75) (end 120 97.5) (width 1.5) (layer B.Cu) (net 3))
 (segment (start 118.75 102.25) (end 118.75 98.75) (width 1.5) (layer B.Cu) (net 3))
 (segment (start 120 97.5) (end 124.75 97.5) (width 1.5) (layer B.Cu) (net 3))
 (segment (start 97.239979 101.239979) (end 101.25 105.25) (width 1.5) (layer B.Cu) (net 3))
 (segment (start 97.239979 100.739979) (end 97.239979 101.239979) (width 1.5) (layer B.Cu) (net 3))
 (segment (start 105.950001 81.700001) (end 105.84998 81.59998) (width 1.5) (layer B.Cu) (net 3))
 (segment (start 110.830001 81.700001) (end 105.950001 81.700001) (width 1.5) (layer B.Cu) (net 3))
 (segment (start 111.63 82.5) (end 110.830001 81.700001) (width 1.5) (layer B.Cu) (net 3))
 (segment (start 142.4032 71.3896) (end 140.2636 69.25) (width 1.2) (layer B.Cu) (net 3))
 (segment (start 142.4032 73.8896) (end 142.4032 71.3896) (width 1.2) (layer B.Cu) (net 3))
 (segment (start 140.2636 69.25) (end 127.75 69.25) (width 1.2) (layer B.Cu) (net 3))
 (segment (start 126.75 70.25) (end 126.75 73) (width 1.2) (layer B.Cu) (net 3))
 (segment (start 127.75 69.25) (end 126.75 70.25) (width 1.2) (layer B.Cu) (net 3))
 (segment (start 125.5 69) (end 126.75 70.25) (width 1.2) (layer B.Cu) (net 3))
 (segment (start 115.25 69) (end 125.5 69) (width 1.2) (layer B.Cu) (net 3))
 (segment (start 114.25 73) (end 114.25 70) (width 1.2) (layer B.Cu) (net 3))
 (segment (start 114.25 70) (end 115.25 69) (width 1.2) (layer B.Cu) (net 3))
 (segment (start 104.24 69) (end 103.25001 69.98999) (width 1.2) (layer B.Cu) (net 3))
 (segment (start 114.25 70) (end 113.25 69) (width 1.2) (layer B.Cu) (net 3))
 (segment (start 113.25 69) (end 104.24 69) (width 1.2) (layer B.Cu) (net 3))
 (segment (start 102.29 89.25) (end 102.29 85.75) (width 1.5) (layer B.Cu) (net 1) (status 30))
 (segment (start 114.17 88.98863) (end 114.17 90.12) (width 1.5) (layer B.Cu) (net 1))
 (segment (start 112.18137 87) (end 114.17 88.98863) (width 1.5) (layer B.Cu) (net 1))
 (segment (start 108.25 87) (end 112.18137 87) (width 1.5) (layer B.Cu) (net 1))
 (segment (start 106 89.25) (end 108.25 87) (width 1.5) (layer B.Cu) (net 1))
 (segment (start 102.29 89.25) (end 106 89.25) (width 1.5) (layer B.Cu) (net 1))
 (segment (start 113.34137 87) (end 112.18137 87) (width 1.5) (layer B.Cu) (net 1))
 (segment (start 116.71 83.63137) (end 113.34137 87) (width 1.5) (layer B.Cu) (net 1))
 (segment (start 116.71 82.5) (end 116.71 83.63137) (width 1.5) (layer B.Cu) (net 1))
 (segment (start 114.17 99.67) (end 115 100.5) (width 1.5) (layer B.Cu) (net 1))
 (segment (start 114.17 90.12) (end 114.17 99.67) (width 1.5) (layer B.Cu) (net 1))
 (segment (start 111.63 90.12) (end 111.63 95.87) (width 1.5) (layer B.Cu) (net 10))
 (segment (start 111.63 95.87) (end 108.5 99) (width 1.5) (layer B.Cu) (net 10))
 (segment (start 130.25 73) (end 134.25 73) (width 1.5) (layer B.Cu) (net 5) (status 10))
 (segment (start 140.2196 78.9696) (end 142.4032 78.9696) (width 1.5) (layer B.Cu) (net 5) (status 20))
 (segment (start 134.25 73) (end 140.2196 78.9696) (width 1.5) (layer B.Cu) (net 5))
 (segment (start 135.1036 76.75) (end 142.4032 84.0496) (width 1.5) (layer B.Cu) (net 6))
 (segment (start 122.75 73) (end 124 74.25) (width 1.5) (layer B.Cu) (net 6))
 (segment (start 117.75 73) (end 122.75 73) (width 1.5) (layer B.Cu) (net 6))
 (segment (start 124 74.25) (end 124 75.5) (width 1.5) (layer B.Cu) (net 6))
 (segment (start 124 75.5) (end 125.25 76.75) (width 1.5) (layer B.Cu) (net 6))
 (segment (start 125.25 76.75) (end 135.1036 76.75) (width 1.5) (layer B.Cu) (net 6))
 (segment (start 107.9 73.04) (end 111.61 76.75) (width 1.5) (layer B.Cu) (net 7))
 (segment (start 105.5 73.04) (end 107.9 73.04) (width 1.5) (layer B.Cu) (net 7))
 (segment (start 111.61 76.75) (end 121.5 76.75) (width 1.5) (layer B.Cu) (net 7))
 (segment (start 121.5 76.75) (end 124 79.25) (width 1.5) (layer B.Cu) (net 7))
 (segment (start 132.5236 79.25) (end 142.4032 89.1296) (width 1.5) (layer B.Cu) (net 7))
 (segment (start 124 79.25) (end 132.5236 79.25) (width 1.5) (layer B.Cu) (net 7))
 (segment (start 114.17 81.36863) (end 116.25 79.28863) (width 1.5) (layer B.Cu) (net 8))
 (segment (start 114.17 82.5) (end 114.17 81.36863) (width 1.5) (layer B.Cu) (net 8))
 (segment (start 116.25 79.28863) (end 120.46137 79.28863) (width 1.5) (layer B.Cu) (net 8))
 (segment (start 120.46137 79.28863) (end 122.67274 81.5) (width 1.5) (layer B.Cu) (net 8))
 (segment (start 129.6936 81.5) (end 142.4032 94.2096) (width 1.5) (layer B.Cu) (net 8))
 (segment (start 122.67274 81.5) (end 129.6936 81.5) (width 1.5) (layer B.Cu) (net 8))
 (segment (start 120.36863 94.25) (end 121.5 94.25) (width 1.5) (layer B.Cu) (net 4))
 (segment (start 119.70863 94.25) (end 120.36863 94.25) (width 1.5) (layer B.Cu) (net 4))
 (segment (start 116.71 91.25137) (end 119.70863 94.25) (width 1.5) (layer B.Cu) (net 4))
 (segment (start 116.71 90.12) (end 116.71 91.25137) (width 1.5) (layer B.Cu) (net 4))
 (segment (start 121.5 94.25) (end 127.5 94.25) (width 1.5) (layer B.Cu) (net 4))
 (segment (start 128.5 95.25) (end 128.5 100.45) (width 1.5) (layer B.Cu) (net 4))
 (segment (start 127.5 94.25) (end 128.5 95.25) (width 1.5) (layer B.Cu) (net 4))
 (segment (start 103.79 94.25) (end 102.29 92.75) (width 1.5) (layer B.Cu) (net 9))
 (segment (start 108.8 94.25) (end 103.79 94.25) (width 1.5) (layer B.Cu) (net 9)))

